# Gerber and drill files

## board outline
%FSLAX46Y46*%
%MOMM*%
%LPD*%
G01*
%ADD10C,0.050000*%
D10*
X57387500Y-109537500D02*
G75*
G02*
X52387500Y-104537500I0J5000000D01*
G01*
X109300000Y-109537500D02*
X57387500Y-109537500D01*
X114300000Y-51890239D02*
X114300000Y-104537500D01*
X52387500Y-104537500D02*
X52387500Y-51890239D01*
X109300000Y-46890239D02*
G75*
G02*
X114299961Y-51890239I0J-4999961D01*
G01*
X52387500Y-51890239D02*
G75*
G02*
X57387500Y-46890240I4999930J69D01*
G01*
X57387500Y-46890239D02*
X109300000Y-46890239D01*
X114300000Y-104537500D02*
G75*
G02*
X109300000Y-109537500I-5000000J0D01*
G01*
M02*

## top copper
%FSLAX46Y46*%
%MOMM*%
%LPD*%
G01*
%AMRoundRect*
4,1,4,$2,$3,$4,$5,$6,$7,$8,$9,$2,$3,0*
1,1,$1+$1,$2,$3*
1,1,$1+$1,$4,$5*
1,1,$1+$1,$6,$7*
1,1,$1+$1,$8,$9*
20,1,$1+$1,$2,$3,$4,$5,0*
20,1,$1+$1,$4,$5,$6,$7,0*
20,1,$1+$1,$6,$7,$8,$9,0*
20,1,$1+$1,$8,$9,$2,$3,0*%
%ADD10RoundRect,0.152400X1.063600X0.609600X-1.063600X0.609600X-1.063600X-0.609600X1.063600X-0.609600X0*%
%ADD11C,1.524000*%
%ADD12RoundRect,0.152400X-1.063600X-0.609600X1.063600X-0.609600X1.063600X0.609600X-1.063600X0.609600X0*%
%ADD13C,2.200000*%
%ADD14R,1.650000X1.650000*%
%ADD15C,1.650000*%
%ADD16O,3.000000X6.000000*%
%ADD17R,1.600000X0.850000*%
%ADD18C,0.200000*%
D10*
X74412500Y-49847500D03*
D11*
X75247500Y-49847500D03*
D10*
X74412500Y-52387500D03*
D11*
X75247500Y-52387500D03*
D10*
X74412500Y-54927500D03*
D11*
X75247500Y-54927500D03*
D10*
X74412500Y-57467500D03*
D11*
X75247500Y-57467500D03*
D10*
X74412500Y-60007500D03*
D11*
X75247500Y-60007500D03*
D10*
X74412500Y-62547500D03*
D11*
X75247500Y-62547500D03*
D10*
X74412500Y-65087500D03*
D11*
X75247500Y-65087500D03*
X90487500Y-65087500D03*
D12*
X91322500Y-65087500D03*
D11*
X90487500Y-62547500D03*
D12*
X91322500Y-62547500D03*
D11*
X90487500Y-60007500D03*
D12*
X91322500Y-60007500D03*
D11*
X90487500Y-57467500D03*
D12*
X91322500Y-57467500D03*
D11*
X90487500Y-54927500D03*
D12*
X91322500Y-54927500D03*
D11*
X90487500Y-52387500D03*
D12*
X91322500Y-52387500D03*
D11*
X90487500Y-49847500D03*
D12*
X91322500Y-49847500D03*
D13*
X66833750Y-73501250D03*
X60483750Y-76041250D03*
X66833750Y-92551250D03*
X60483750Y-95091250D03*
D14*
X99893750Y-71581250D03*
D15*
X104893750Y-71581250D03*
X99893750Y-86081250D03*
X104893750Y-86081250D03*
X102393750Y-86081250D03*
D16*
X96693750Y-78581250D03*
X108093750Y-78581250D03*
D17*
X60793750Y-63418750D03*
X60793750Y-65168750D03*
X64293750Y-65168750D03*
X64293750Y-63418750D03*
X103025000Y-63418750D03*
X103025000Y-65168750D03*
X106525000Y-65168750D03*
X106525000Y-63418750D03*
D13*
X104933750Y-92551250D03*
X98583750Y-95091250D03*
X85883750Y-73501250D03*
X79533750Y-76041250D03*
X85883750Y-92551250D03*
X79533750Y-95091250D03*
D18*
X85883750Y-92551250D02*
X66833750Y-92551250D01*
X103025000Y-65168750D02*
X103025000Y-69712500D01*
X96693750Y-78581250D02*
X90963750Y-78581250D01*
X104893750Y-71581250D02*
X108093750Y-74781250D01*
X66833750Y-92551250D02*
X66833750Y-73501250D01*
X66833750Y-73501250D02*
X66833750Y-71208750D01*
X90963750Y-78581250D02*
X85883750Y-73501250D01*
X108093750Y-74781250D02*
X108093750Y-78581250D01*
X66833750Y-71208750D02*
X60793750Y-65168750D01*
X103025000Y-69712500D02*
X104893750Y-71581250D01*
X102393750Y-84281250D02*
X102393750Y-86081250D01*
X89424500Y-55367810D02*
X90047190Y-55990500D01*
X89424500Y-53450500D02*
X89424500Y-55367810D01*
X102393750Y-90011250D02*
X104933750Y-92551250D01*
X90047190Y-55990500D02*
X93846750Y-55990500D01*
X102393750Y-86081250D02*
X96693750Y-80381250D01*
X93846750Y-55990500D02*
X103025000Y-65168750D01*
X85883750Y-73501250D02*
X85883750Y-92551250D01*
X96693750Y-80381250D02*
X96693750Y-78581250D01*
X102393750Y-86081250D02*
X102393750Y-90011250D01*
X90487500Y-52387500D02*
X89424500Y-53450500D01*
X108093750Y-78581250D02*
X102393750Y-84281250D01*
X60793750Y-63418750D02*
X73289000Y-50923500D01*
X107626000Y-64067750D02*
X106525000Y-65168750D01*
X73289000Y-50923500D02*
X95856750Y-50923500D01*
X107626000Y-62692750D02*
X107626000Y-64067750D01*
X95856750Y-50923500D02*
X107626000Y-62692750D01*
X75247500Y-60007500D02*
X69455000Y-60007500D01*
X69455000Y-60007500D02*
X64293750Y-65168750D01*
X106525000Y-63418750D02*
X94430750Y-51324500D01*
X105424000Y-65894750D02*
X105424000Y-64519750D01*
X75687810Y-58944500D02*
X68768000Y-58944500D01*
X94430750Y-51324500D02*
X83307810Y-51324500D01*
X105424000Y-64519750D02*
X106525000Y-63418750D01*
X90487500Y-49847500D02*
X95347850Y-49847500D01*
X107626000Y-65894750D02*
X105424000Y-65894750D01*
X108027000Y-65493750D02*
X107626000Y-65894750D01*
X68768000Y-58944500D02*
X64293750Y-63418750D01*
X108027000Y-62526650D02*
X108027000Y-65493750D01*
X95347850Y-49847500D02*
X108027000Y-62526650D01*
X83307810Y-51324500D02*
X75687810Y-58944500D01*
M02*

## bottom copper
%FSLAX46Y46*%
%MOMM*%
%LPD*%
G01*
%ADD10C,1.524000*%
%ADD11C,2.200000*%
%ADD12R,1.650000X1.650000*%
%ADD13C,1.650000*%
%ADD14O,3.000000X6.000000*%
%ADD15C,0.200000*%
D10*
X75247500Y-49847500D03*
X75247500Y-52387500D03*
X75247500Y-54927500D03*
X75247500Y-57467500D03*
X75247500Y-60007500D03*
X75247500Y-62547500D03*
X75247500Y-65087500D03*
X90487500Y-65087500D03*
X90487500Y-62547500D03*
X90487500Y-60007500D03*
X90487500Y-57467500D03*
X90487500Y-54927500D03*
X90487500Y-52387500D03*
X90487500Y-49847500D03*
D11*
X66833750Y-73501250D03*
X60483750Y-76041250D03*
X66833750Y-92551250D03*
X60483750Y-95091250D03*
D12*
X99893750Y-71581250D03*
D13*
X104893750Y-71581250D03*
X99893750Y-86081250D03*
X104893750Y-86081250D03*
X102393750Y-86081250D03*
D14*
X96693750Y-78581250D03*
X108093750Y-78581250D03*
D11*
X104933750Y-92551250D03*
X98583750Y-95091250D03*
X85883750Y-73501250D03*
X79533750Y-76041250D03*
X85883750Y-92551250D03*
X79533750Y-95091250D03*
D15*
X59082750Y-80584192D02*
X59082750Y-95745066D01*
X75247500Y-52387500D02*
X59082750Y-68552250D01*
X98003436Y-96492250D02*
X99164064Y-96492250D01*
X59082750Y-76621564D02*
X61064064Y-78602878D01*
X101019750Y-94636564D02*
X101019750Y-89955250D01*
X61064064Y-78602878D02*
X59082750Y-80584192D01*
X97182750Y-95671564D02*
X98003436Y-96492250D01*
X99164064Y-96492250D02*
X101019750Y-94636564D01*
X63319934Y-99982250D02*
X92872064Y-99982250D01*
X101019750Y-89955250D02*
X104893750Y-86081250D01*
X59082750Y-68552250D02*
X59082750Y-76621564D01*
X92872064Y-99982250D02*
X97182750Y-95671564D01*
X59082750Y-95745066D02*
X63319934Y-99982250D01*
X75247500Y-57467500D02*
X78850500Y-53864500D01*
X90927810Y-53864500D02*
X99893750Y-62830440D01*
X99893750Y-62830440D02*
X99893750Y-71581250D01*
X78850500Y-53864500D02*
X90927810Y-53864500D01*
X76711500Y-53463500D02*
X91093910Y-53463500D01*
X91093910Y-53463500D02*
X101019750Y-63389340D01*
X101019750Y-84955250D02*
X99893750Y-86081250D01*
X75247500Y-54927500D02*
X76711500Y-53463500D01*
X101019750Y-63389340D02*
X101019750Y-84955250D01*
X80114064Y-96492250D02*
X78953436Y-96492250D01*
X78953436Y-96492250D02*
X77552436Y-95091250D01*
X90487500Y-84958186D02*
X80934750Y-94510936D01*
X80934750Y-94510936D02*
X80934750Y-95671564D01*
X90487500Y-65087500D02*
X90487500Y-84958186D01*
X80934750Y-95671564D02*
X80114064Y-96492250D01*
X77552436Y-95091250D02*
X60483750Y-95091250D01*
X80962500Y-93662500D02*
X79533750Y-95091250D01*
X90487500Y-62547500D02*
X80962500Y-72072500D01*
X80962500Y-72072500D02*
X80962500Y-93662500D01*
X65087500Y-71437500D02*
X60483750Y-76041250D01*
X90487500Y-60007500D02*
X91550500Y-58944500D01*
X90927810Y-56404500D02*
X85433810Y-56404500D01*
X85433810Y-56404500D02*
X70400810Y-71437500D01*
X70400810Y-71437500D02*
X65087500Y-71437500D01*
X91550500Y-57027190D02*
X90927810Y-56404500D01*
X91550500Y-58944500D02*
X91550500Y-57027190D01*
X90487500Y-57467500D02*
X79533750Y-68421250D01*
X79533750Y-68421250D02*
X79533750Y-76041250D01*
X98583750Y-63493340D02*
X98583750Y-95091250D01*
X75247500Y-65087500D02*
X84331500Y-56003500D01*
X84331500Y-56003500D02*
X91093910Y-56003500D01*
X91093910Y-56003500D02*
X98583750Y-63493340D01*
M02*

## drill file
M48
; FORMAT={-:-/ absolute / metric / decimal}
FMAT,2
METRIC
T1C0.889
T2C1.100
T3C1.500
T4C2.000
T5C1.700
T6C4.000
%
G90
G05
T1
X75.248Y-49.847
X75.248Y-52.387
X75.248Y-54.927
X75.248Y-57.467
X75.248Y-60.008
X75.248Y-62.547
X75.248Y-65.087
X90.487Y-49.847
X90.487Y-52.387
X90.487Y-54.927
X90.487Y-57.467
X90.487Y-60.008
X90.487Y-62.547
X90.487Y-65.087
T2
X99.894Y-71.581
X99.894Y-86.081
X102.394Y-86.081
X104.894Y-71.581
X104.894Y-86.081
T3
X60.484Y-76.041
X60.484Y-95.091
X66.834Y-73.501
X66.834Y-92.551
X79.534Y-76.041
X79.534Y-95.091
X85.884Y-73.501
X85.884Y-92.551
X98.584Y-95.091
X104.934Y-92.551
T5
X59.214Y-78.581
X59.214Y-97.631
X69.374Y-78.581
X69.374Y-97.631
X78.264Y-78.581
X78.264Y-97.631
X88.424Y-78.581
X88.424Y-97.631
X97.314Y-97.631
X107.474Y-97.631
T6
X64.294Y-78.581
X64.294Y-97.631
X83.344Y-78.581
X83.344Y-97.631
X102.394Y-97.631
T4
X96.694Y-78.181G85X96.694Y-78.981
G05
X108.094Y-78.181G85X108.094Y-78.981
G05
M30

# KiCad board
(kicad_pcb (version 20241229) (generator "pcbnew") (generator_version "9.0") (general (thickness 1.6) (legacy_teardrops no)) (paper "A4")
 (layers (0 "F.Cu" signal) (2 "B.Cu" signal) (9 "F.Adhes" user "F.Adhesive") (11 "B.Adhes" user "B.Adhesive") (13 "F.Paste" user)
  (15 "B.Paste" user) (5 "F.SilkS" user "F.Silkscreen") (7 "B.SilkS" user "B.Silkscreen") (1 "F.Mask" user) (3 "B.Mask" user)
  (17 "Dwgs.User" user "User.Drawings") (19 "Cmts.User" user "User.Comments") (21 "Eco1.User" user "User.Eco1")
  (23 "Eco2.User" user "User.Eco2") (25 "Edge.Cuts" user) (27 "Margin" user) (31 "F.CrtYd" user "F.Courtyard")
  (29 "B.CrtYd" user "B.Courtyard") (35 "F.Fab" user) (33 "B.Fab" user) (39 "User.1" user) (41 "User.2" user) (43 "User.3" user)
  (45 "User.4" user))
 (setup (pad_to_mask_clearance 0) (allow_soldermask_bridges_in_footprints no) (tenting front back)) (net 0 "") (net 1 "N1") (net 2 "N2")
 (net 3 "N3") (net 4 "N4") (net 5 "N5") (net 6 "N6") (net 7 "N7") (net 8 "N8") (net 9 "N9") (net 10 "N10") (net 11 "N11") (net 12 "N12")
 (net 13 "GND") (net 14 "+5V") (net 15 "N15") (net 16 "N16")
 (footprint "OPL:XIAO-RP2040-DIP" (layer "F.Cu") (at 82.8675 57.4675)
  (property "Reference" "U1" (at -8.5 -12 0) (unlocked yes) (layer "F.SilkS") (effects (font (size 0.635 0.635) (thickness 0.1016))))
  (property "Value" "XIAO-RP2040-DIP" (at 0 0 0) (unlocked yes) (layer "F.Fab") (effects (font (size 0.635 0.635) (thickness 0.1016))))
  (pad "1" smd roundrect (at -8.455 -7.62 180) (size 2.432 1.524) (layers "F.Cu" "F.Mask") (roundrect_rratio 0.1) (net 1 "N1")
   (thermal_bridge_angle 45))
  (pad "1" thru_hole circle (at -7.62 -7.62 180) (size 1.524 1.524) (drill 0.889) (layers "*.Cu" "*.Mask") (remove_unused_layers no)
   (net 1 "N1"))
  (pad "2" smd roundrect (at -8.455 -5.08 180) (size 2.432 1.524) (layers "F.Cu" "F.Mask") (roundrect_rratio 0.1) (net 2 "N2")
   (thermal_bridge_angle 45))
  (pad "2" thru_hole circle (at -7.62 -5.08 180) (size 1.524 1.524) (drill 0.889) (layers "*.Cu" "*.Mask") (remove_unused_layers no)
   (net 2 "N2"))
  (pad "3" smd roundrect (at -8.455 -2.54 180) (size 2.432 1.524) (layers "F.Cu" "F.Mask") (roundrect_rratio 0.1) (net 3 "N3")
   (thermal_bridge_angle 45))
  (pad "3" thru_hole circle (at -7.62 -2.54 180) (size 1.524 1.524) (drill 0.889) (layers "*.Cu" "*.Mask") (remove_unused_layers no)
   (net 3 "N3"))
  (pad "4" smd roundrect (at -8.455 0 180) (size 2.432 1.524) (layers "F.Cu" "F.Mask") (roundrect_rratio 0.1) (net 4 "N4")
   (thermal_bridge_angle 45))
  (pad "4" thru_hole circle (at -7.62 0 180) (size 1.524 1.524) (drill 0.889) (layers "*.Cu" "*.Mask") (remove_unused_layers no)
   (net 4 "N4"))
  (pad "5" smd roundrect (at -8.455 2.54 180) (size 2.432 1.524) (layers "F.Cu" "F.Mask") (roundrect_rratio 0.1) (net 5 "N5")
   (thermal_bridge_angle 45))
  (pad "5" thru_hole circle (at -7.62 2.54 180) (size 1.524 1.524) (drill 0.889) (layers "*.Cu" "*.Mask") (remove_unused_layers no)
   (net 5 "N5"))
  (pad "6" smd roundrect (at -8.455 5.08 180) (size 2.432 1.524) (layers "F.Cu" "F.Mask") (roundrect_rratio 0.1) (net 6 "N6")
   (thermal_bridge_angle 45))
  (pad "6" thru_hole circle (at -7.62 5.08 180) (size 1.524 1.524) (drill 0.889) (layers "*.Cu" "*.Mask") (remove_unused_layers no)
   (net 6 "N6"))
  (pad "7" smd roundrect (at -8.455 7.62 180) (size 2.432 1.524) (layers "F.Cu" "F.Mask") (roundrect_rratio 0.1) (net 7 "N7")
   (thermal_bridge_angle 45))
  (pad "7" thru_hole circle (at -7.62 7.62 180) (size 1.524 1.524) (drill 0.889) (layers "*.Cu" "*.Mask") (remove_unused_layers no)
   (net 7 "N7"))
  (pad "8" thru_hole circle (at 7.62 7.62) (size 1.524 1.524) (drill 0.889) (layers "*.Cu" "*.Mask") (remove_unused_layers no) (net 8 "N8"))
  (pad "8" smd roundrect (at 8.455 7.62) (size 2.432 1.524) (layers "F.Cu" "F.Mask") (roundrect_rratio 0.1) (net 8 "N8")
   (thermal_bridge_angle 45))
  (pad "9" thru_hole circle (at 7.62 5.08) (size 1.524 1.524) (drill 0.889) (layers "*.Cu" "*.Mask") (remove_unused_layers no) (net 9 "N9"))
  (pad "9" smd roundrect (at 8.455 5.08) (size 2.432 1.524) (layers "F.Cu" "F.Mask") (roundrect_rratio 0.1) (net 9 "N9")
   (thermal_bridge_angle 45))
  (pad "10" thru_hole circle (at 7.62 2.54) (size 1.524 1.524) (drill 0.889) (layers "*.Cu" "*.Mask") (remove_unused_layers no)
   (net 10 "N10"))
  (pad "10" smd roundrect (at 8.455 2.54) (size 2.432 1.524) (layers "F.Cu" "F.Mask") (roundrect_rratio 0.1) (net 10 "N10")
   (thermal_bridge_angle 45))
  (pad "11" thru_hole circle (at 7.62 0) (size 1.524 1.524) (drill 0.889) (layers "*.Cu" "*.Mask") (remove_unused_layers no) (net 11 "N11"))
  (pad "11" smd roundrect (at 8.455 0) (size 2.432 1.524) (layers "F.Cu" "F.Mask") (roundrect_rratio 0.1) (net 11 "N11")
   (thermal_bridge_angle 45))
  (pad "12" thru_hole circle (at 7.62 -2.54) (size 1.524 1.524) (drill 0.889) (layers "*.Cu" "*.Mask") (remove_unused_layers no)
   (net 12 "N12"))
  (pad "12" smd roundrect (at 8.455 -2.54) (size 2.432 1.524) (layers "F.Cu" "F.Mask") (roundrect_rratio 0.1) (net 12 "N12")
   (thermal_bridge_angle 45))
  (pad "13" thru_hole circle (at 7.62 -5.08) (size 1.524 1.524) (drill 0.889) (layers "*.Cu" "*.Mask") (remove_unused_layers no)
   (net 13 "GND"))
  (pad "13" smd roundrect (at 8.455 -5.08) (size 2.432 1.524) (layers "F.Cu" "F.Mask") (roundrect_rratio 0.1) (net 13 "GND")
   (thermal_bridge_angle 45))
  (pad "14" thru_hole circle (at 7.62 -7.62) (size 1.524 1.524) (drill 0.889) (layers "*.Cu" "*.Mask") (remove_unused_layers no)
   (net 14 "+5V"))
  (pad "14" smd roundrect (at 8.455 -7.62) (size 2.432 1.524) (layers "F.Cu" "F.Mask") (roundrect_rratio 0.1) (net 14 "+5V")
   (thermal_bridge_angle 45)))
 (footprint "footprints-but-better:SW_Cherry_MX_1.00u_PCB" (layer "F.Cu") (at 66.83375 73.50125)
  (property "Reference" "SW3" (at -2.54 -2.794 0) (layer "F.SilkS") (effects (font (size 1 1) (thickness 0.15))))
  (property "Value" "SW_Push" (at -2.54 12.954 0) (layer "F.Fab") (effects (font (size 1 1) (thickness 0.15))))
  (pad "" np_thru_hole circle (at -7.62 5.08) (size 1.7 1.7) (drill 1.7) (layers "*.Cu" "*.Mask"))
  (pad "" np_thru_hole circle (at -2.54 5.08) (size 4 4) (drill 4) (layers "*.Cu" "*.Mask"))
  (pad "" np_thru_hole circle (at 2.54 5.08) (size 1.7 1.7) (drill 1.7) (layers "*.Cu" "*.Mask"))
  (pad "1" thru_hole circle (at 0 0) (size 2.2 2.2) (drill 1.5) (layers "*.Cu" "*.Mask") (remove_unused_layers no) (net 13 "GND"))
  (pad "2" thru_hole circle (at -6.35 2.54) (size 2.2 2.2) (drill 1.5) (layers "*.Cu" "*.Mask") (remove_unused_layers no) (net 10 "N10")))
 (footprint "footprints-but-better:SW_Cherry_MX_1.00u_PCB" (layer "F.Cu") (at 66.83375 92.55125)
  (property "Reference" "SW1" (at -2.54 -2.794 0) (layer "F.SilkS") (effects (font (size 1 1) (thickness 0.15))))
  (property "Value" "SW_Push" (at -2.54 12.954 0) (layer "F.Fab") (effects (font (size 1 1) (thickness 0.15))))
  (pad "" np_thru_hole circle (at -7.62 5.08) (size 1.7 1.7) (drill 1.7) (layers "*.Cu" "*.Mask"))
  (pad "" np_thru_hole circle (at -2.54 5.08) (size 4 4) (drill 4) (layers "*.Cu" "*.Mask"))
  (pad "" np_thru_hole circle (at 2.54 5.08) (size 1.7 1.7) (drill 1.7) (layers "*.Cu" "*.Mask"))
  (pad "1" thru_hole circle (at 0 0) (size 2.2 2.2) (drill 1.5) (layers "*.Cu" "*.Mask") (remove_unused_layers no) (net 13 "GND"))
  (pad "2" thru_hole circle (at -6.35 2.54) (size 2.2 2.2) (drill 1.5) (layers "*.Cu" "*.Mask") (remove_unused_layers no) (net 8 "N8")))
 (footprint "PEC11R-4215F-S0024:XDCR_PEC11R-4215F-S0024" (layer "F.Cu") (at 102.39375 78.58125)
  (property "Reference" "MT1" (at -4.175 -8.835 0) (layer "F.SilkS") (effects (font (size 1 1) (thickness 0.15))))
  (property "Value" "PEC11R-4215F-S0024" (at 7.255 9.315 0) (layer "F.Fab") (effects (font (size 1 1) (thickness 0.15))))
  (pad "1" thru_hole rect (at -2.5 -7) (size 1.65 1.65) (drill 1.1) (layers "*.Cu" "*.Mask") (remove_unused_layers no) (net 4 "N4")
   (solder_mask_margin 0.102))
  (pad "2" thru_hole circle (at 2.5 -7) (size 1.65 1.65) (drill 1.1) (layers "*.Cu" "*.Mask") (remove_unused_layers no) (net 13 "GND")
   (solder_mask_margin 0.102))
  (pad "A" thru_hole circle (at -2.5 7.5) (size 1.65 1.65) (drill 1.1) (layers "*.Cu" "*.Mask") (remove_unused_layers no) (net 3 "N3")
   (solder_mask_margin 0.102))
  (pad "B" thru_hole circle (at 2.5 7.5) (size 1.65 1.65) (drill 1.1) (layers "*.Cu" "*.Mask") (remove_unused_layers no) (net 2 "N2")
   (solder_mask_margin 0.102))
  (pad "COM" thru_hole circle (at 0 7.5) (size 1.65 1.65) (drill 1.1) (layers "*.Cu" "*.Mask") (remove_unused_layers no) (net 13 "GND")
   (solder_mask_margin 0.102))
  (pad "S1" thru_hole oval (at -5.7 0) (size 3 6) (drill oval 2 2.8) (layers "*.Cu" "*.Mask") (remove_unused_layers no) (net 13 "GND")
   (solder_mask_margin 0.102))
  (pad "S2" thru_hole oval (at 5.7 0) (size 3 6) (drill oval 2 2.8) (layers "*.Cu" "*.Mask") (remove_unused_layers no) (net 13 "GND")
   (solder_mask_margin 0.102)))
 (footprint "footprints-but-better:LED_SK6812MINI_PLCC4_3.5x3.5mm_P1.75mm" (layer "F.Cu") (at 62.54375 64.29375)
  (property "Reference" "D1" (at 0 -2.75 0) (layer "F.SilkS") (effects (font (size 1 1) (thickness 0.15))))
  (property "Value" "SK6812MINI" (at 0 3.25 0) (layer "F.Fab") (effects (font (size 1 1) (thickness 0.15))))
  (pad "1" smd rect (at -1.75 -0.875) (size 1.6 0.85) (layers "F.Cu" "F.Mask" "F.Paste") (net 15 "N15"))
  (pad "2" smd rect (at -1.75 0.875) (size 1.6 0.85) (layers "F.Cu" "F.Mask" "F.Paste") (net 13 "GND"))
  (pad "3" smd rect (at 1.75 0.875) (size 1.6 0.85) (layers "F.Cu" "F.Mask" "F.Paste") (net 5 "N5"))
  (pad "4" smd rect (at 1.75 -0.875) (size 1.6 0.85) (layers "F.Cu" "F.Mask" "F.Paste") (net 14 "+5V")))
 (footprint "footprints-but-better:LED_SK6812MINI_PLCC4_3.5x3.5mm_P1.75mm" (layer "F.Cu") (at 104.775 64.29375)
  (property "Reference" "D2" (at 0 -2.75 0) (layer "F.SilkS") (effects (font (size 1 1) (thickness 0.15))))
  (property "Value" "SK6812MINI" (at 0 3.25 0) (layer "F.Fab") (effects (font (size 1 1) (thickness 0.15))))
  (pad "1" smd rect (at -1.75 -0.875) (size 1.6 0.85) (layers "F.Cu" "F.Mask" "F.Paste") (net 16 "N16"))
  (pad "2" smd rect (at -1.75 0.875) (size 1.6 0.85) (layers "F.Cu" "F.Mask" "F.Paste") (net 13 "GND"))
  (pad "3" smd rect (at 1.75 0.875) (size 1.6 0.85) (layers "F.Cu" "F.Mask" "F.Paste") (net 15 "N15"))
  (pad "4" smd rect (at 1.75 -0.875) (size 1.6 0.85) (layers "F.Cu" "F.Mask" "F.Paste") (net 14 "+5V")))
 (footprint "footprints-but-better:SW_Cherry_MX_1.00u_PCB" (layer "F.Cu") (at 104.93375 92.55125)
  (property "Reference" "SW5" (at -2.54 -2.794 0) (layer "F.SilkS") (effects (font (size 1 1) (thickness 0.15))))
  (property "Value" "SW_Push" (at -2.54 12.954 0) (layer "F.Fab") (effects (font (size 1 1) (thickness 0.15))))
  (pad "" np_thru_hole circle (at -7.62 5.08) (size 1.7 1.7) (drill 1.7) (layers "*.Cu" "*.Mask"))
  (pad "" np_thru_hole circle (at -2.54 5.08) (size 4 4) (drill 4) (layers "*.Cu" "*.Mask"))
  (pad "" np_thru_hole circle (at 2.54 5.08) (size 1.7 1.7) (drill 1.7) (layers "*.Cu" "*.Mask"))
  (pad "1" thru_hole circle (at 0 0) (size 2.2 2.2) (drill 1.5) (layers "*.Cu" "*.Mask") (remove_unused_layers no) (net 13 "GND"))
  (pad "2" thru_hole circle (at -6.35 2.54) (size 2.2 2.2) (drill 1.5) (layers "*.Cu" "*.Mask") (remove_unused_layers no) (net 7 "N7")))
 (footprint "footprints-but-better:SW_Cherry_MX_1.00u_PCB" (layer "F.Cu") (at 85.88375 73.50125)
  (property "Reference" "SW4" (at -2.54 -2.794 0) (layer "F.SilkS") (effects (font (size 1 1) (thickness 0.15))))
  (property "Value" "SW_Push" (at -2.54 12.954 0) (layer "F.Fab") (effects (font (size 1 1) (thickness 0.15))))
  (pad "" np_thru_hole circle (at -7.62 5.08) (size 1.7 1.7) (drill 1.7) (layers "*.Cu" "*.Mask"))
  (pad "" np_thru_hole circle (at -2.54 5.08) (size 4 4) (drill 4) (layers "*.Cu" "*.Mask"))
  (pad "" np_thru_hole circle (at 2.54 5.08) (size 1.7 1.7) (drill 1.7) (layers "*.Cu" "*.Mask"))
  (pad "1" thru_hole circle (at 0 0) (size 2.2 2.2) (drill 1.5) (layers "*.Cu" "*.Mask") (remove_unused_layers no) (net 13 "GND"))
  (pad "2" thru_hole circle (at -6.35 2.54) (size 2.2 2.2) (drill 1.5) (layers "*.Cu" "*.Mask") (remove_unused_layers no) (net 11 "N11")))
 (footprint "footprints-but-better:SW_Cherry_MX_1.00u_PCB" (layer "F.Cu") (at 85.88375 92.55125)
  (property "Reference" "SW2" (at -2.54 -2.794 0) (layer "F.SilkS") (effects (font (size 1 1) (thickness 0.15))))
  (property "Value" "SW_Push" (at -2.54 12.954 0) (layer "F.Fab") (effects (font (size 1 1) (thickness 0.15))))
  (pad "" np_thru_hole circle (at -7.62 5.08) (size 1.7 1.7) (drill 1.7) (layers "*.Cu" "*.Mask"))
  (pad "" np_thru_hole circle (at -2.54 5.08) (size 4 4) (drill 4) (layers "*.Cu" "*.Mask"))
  (pad "" np_thru_hole circle (at 2.54 5.08) (size 1.7 1.7) (drill 1.7) (layers "*.Cu" "*.Mask"))
  (pad "1" thru_hole circle (at 0 0) (size 2.2 2.2) (drill 1.5) (layers "*.Cu" "*.Mask") (remove_unused_layers no) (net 13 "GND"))
  (pad "2" thru_hole circle (at -6.35 2.54) (size 2.2 2.2) (drill 1.5) (layers "*.Cu" "*.Mask") (remove_unused_layers no) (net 9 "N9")))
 (gr_arc (start 57.3875 109.5375) (mid 53.851966 108.073034) (end 52.3875 104.5375) (stroke (width 0.05) (type default)) (layer "Edge.Cuts"))
 (gr_line (start 109.3 109.5375) (end 57.3875 109.5375) (stroke (width 0.05) (type default)) (layer "Edge.Cuts"))
 (gr_line (start 114.3 51.890239) (end 114.3 104.5375) (stroke (width 0.05) (type default)) (layer "Edge.Cuts"))
 (gr_line (start 52.3875 104.5375) (end 52.3875 51.890239) (stroke (width 0.05) (type default)) (layer "Edge.Cuts"))
 (gr_arc (start 109.3 46.890239) (mid 112.835534 48.354705) (end 114.3 51.890239) (stroke (width 0.05) (type default)) (layer "Edge.Cuts"))
 (gr_arc (start 52.3875 51.890239) (mid 53.851952 48.35468) (end 57.3875 46.890239) (stroke (width 0.05) (type default)) (layer "Edge.Cuts"))
 (gr_line (start 57.3875 46.890239) (end 109.3 46.890239) (stroke (width 0.05) (type default)) (layer "Edge.Cuts"))
 (gr_arc (start 114.3 104.5375) (mid 112.835534 108.073034) (end 109.3 109.5375) (stroke (width 0.05) (type default)) (layer "Edge.Cuts"))
 (segment (start 85.88375 92.55125) (end 66.83375 92.55125) (width 0.2) (layer "F.Cu") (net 13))
 (segment (start 103.025 65.16875) (end 103.025 69.7125) (width 0.2) (layer "F.Cu") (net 13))
 (segment (start 96.69375 78.58125) (end 90.96375 78.58125) (width 0.2) (layer "F.Cu") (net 13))
 (segment (start 104.89375 71.58125) (end 108.09375 74.78125) (width 0.2) (layer "F.Cu") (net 13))
 (segment (start 66.83375 92.55125) (end 66.83375 73.50125) (width 0.2) (layer "F.Cu") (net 13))
 (segment (start 66.83375 73.50125) (end 66.83375 71.20875) (width 0.2) (layer "F.Cu") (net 13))
 (segment (start 90.96375 78.58125) (end 85.88375 73.50125) (width 0.2) (layer "F.Cu") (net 13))
 (segment (start 108.09375 74.78125) (end 108.09375 78.58125) (width 0.2) (layer "F.Cu") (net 13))
 (segment (start 66.83375 71.20875) (end 60.79375 65.16875) (width 0.2) (layer "F.Cu") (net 13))
 (segment (start 103.025 69.7125) (end 104.89375 71.58125) (width 0.2) (layer "F.Cu") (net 13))
 (segment (start 102.39375 84.28125) (end 102.39375 86.08125) (width 0.2) (layer "F.Cu") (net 13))
 (segment (start 89.4245 55.36781) (end 90.04719 55.9905) (width 0.2) (layer "F.Cu") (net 13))
 (segment (start 89.4245 53.4505) (end 89.4245 55.36781) (width 0.2) (layer "F.Cu") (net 13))
 (segment (start 102.39375 90.01125) (end 104.93375 92.55125) (width 0.2) (layer "F.Cu") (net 13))
 (segment (start 90.04719 55.9905) (end 93.84675 55.9905) (width 0.2) (layer "F.Cu") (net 13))
 (segment (start 102.39375 86.08125) (end 96.69375 80.38125) (width 0.2) (layer "F.Cu") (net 13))
 (segment (start 93.84675 55.9905) (end 103.025 65.16875) (width 0.2) (layer "F.Cu") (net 13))
 (segment (start 85.88375 73.50125) (end 85.88375 92.55125) (width 0.2) (layer "F.Cu") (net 13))
 (segment (start 96.69375 80.38125) (end 96.69375 78.58125) (width 0.2) (layer "F.Cu") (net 13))
 (segment (start 102.39375 86.08125) (end 102.39375 90.01125) (width 0.2) (layer "F.Cu") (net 13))
 (segment (start 90.4875 52.3875) (end 89.4245 53.4505) (width 0.2) (layer "F.Cu") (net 13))
 (segment (start 108.09375 78.58125) (end 102.39375 84.28125) (width 0.2) (layer "F.Cu") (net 13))
 (segment (start 60.79375 63.41875) (end 73.289 50.9235) (width 0.2) (layer "F.Cu") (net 15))
 (segment (start 107.626 64.06775) (end 106.525 65.16875) (width 0.2) (layer "F.Cu") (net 15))
 (segment (start 73.289 50.9235) (end 95.85675 50.9235) (width 0.2) (layer "F.Cu") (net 15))
 (segment (start 107.626 62.69275) (end 107.626 64.06775) (width 0.2) (layer "F.Cu") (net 15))
 (segment (start 95.85675 50.9235) (end 107.626 62.69275) (width 0.2) (layer "F.Cu") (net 15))
 (segment (start 75.2475 60.0075) (end 69.455 60.0075) (width 0.2) (layer "F.Cu") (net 5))
 (segment (start 69.455 60.0075) (end 64.29375 65.16875) (width 0.2) (layer "F.Cu") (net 5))
 (segment (start 59.08275 80.584192) (end 59.08275 95.745066) (width 0.2) (layer "B.Cu") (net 2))
 (segment (start 75.2475 52.3875) (end 59.08275 68.55225) (width 0.2) (layer "B.Cu") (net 2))
 (segment (start 98.003436 96.49225) (end 99.164064 96.49225) (width 0.2) (layer "B.Cu") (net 2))
 (segment (start 59.08275 76.621564) (end 61.064064 78.602878) (width 0.2) (layer "B.Cu") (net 2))
 (segment (start 101.01975 94.636564) (end 101.01975 89.95525) (width 0.2) (layer "B.Cu") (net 2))
 (segment (start 61.064064 78.602878) (end 59.08275 80.584192) (width 0.2) (layer "B.Cu") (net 2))
 (segment (start 97.18275 95.671564) (end 98.003436 96.49225) (width 0.2) (layer "B.Cu") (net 2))
 (segment (start 99.164064 96.49225) (end 101.01975 94.636564) (width 0.2) (layer "B.Cu") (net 2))
 (segment (start 63.319934 99.98225) (end 92.872064 99.98225) (width 0.2) (layer "B.Cu") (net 2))
 (segment (start 101.01975 89.95525) (end 104.89375 86.08125) (width 0.2) (layer "B.Cu") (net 2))
 (segment (start 59.08275 68.55225) (end 59.08275 76.621564) (width 0.2) (layer "B.Cu") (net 2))
 (segment (start 92.872064 99.98225) (end 97.18275 95.671564) (width 0.2) (layer "B.Cu") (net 2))
 (segment (start 59.08275 95.745066) (end 63.319934 99.98225) (width 0.2) (layer "B.Cu") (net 2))
 (segment (start 75.2475 57.4675) (end 78.8505 53.8645) (width 0.2) (layer "B.Cu") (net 4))
 (segment (start 90.92781 53.8645) (end 99.89375 62.83044) (width 0.2) (layer "B.Cu") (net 4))
 (segment (start 99.89375 62.83044) (end 99.89375 71.58125) (width 0.2) (layer "B.Cu") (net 4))
 (segment (start 78.8505 53.8645) (end 90.92781 53.8645) (width 0.2) (layer "B.Cu") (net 4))
 (segment (start 76.7115 53.4635) (end 91.09391 53.4635) (width 0.2) (layer "B.Cu") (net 3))
 (segment (start 91.09391 53.4635) (end 101.01975 63.38934) (width 0.2) (layer "B.Cu") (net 3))
 (segment (start 101.01975 84.95525) (end 99.89375 86.08125) (width 0.2) (layer "B.Cu") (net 3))
 (segment (start 75.2475 54.9275) (end 76.7115 53.4635) (width 0.2) (layer "B.Cu") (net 3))
 (segment (start 101.01975 63.38934) (end 101.01975 84.95525) (width 0.2) (layer "B.Cu") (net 3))
 (segment (start 80.114064 96.49225) (end 78.953436 96.49225) (width 0.2) (layer "B.Cu") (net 8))
 (segment (start 78.953436 96.49225) (end 77.552436 95.09125) (width 0.2) (layer "B.Cu") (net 8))
 (segment (start 90.4875 84.958186) (end 80.93475 94.510936) (width 0.2) (layer "B.Cu") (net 8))
 (segment (start 80.93475 94.510936) (end 80.93475 95.671564) (width 0.2) (layer "B.Cu") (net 8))
 (segment (start 90.4875 65.0875) (end 90.4875 84.958186) (width 0.2) (layer "B.Cu") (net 8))
 (segment (start 80.93475 95.671564) (end 80.114064 96.49225) (width 0.2) (layer "B.Cu") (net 8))
 (segment (start 77.552436 95.09125) (end 60.48375 95.09125) (width 0.2) (layer "B.Cu") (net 8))
 (segment (start 80.9625 93.6625) (end 79.53375 95.09125) (width 0.2) (layer "B.Cu") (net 9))
 (segment (start 90.4875 62.5475) (end 80.9625 72.0725) (width 0.2) (layer "B.Cu") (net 9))
 (segment (start 80.9625 72.0725) (end 80.9625 93.6625) (width 0.2) (layer "B.Cu") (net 9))
 (segment (start 65.0875 71.4375) (end 60.48375 76.04125) (width 0.2) (layer "B.Cu") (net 10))
 (segment (start 90.4875 60.0075) (end 91.5505 58.9445) (width 0.2) (layer "B.Cu") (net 10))
 (segment (start 90.92781 56.4045) (end 85.43381 56.4045) (width 0.2) (layer "B.Cu") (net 10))
 (segment (start 85.43381 56.4045) (end 70.40081 71.4375) (width 0.2) (layer "B.Cu") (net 10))
 (segment (start 70.40081 71.4375) (end 65.0875 71.4375) (width 0.2) (layer "B.Cu") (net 10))
 (segment (start 91.5505 57.02719) (end 90.92781 56.4045) (width 0.2) (layer "B.Cu") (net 10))
 (segment (start 91.5505 58.9445) (end 91.5505 57.02719) (width 0.2) (layer "B.Cu") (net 10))
 (segment (start 90.4875 57.4675) (end 79.53375 68.42125) (width 0.2) (layer "B.Cu") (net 11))
 (segment (start 79.53375 68.42125) (end 79.53375 76.04125) (width 0.2) (layer "B.Cu") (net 11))
 (segment (start 98.58375 63.49334) (end 98.58375 95.09125) (width 0.2) (layer "B.Cu") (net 7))
 (segment (start 75.2475 65.0875) (end 84.3315 56.0035) (width 0.2) (layer "B.Cu") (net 7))
 (segment (start 84.3315 56.0035) (end 91.09391 56.0035) (width 0.2) (layer "B.Cu") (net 7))
 (segment (start 91.09391 56.0035) (end 98.58375 63.49334) (width 0.2) (layer "B.Cu") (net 7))
 (segment (start 106.525 63.41875) (end 94.43075 51.3245) (width 0.2) (layer "F.Cu") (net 14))
 (segment (start 105.424 65.89475) (end 105.424 64.51975) (width 0.2) (layer "F.Cu") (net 14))
 (segment (start 75.68781 58.9445) (end 68.768 58.9445) (width 0.2) (layer "F.Cu") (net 14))
 (segment (start 94.43075 51.3245) (end 83.30781 51.3245) (width 0.2) (layer "F.Cu") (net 14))
 (segment (start 105.424 64.51975) (end 106.525 63.41875) (width 0.2) (layer "F.Cu") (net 14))
 (segment (start 90.4875 49.8475) (end 95.34785 49.8475) (width 0.2) (layer "F.Cu") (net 14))
 (segment (start 107.626 65.89475) (end 105.424 65.89475) (width 0.2) (layer "F.Cu") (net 14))
 (segment (start 108.027 65.49375) (end 107.626 65.89475) (width 0.2) (layer "F.Cu") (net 14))
 (segment (start 68.768 58.9445) (end 64.29375 63.41875) (width 0.2) (layer "F.Cu") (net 14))
 (segment (start 108.027 62.52665) (end 108.027 65.49375) (width 0.2) (layer "F.Cu") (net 14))
 (segment (start 95.34785 49.8475) (end 108.027 62.52665) (width 0.2) (layer "F.Cu") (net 14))
 (segment (start 83.30781 51.3245) (end 75.68781 58.9445) (width 0.2) (layer "F.Cu") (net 14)))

